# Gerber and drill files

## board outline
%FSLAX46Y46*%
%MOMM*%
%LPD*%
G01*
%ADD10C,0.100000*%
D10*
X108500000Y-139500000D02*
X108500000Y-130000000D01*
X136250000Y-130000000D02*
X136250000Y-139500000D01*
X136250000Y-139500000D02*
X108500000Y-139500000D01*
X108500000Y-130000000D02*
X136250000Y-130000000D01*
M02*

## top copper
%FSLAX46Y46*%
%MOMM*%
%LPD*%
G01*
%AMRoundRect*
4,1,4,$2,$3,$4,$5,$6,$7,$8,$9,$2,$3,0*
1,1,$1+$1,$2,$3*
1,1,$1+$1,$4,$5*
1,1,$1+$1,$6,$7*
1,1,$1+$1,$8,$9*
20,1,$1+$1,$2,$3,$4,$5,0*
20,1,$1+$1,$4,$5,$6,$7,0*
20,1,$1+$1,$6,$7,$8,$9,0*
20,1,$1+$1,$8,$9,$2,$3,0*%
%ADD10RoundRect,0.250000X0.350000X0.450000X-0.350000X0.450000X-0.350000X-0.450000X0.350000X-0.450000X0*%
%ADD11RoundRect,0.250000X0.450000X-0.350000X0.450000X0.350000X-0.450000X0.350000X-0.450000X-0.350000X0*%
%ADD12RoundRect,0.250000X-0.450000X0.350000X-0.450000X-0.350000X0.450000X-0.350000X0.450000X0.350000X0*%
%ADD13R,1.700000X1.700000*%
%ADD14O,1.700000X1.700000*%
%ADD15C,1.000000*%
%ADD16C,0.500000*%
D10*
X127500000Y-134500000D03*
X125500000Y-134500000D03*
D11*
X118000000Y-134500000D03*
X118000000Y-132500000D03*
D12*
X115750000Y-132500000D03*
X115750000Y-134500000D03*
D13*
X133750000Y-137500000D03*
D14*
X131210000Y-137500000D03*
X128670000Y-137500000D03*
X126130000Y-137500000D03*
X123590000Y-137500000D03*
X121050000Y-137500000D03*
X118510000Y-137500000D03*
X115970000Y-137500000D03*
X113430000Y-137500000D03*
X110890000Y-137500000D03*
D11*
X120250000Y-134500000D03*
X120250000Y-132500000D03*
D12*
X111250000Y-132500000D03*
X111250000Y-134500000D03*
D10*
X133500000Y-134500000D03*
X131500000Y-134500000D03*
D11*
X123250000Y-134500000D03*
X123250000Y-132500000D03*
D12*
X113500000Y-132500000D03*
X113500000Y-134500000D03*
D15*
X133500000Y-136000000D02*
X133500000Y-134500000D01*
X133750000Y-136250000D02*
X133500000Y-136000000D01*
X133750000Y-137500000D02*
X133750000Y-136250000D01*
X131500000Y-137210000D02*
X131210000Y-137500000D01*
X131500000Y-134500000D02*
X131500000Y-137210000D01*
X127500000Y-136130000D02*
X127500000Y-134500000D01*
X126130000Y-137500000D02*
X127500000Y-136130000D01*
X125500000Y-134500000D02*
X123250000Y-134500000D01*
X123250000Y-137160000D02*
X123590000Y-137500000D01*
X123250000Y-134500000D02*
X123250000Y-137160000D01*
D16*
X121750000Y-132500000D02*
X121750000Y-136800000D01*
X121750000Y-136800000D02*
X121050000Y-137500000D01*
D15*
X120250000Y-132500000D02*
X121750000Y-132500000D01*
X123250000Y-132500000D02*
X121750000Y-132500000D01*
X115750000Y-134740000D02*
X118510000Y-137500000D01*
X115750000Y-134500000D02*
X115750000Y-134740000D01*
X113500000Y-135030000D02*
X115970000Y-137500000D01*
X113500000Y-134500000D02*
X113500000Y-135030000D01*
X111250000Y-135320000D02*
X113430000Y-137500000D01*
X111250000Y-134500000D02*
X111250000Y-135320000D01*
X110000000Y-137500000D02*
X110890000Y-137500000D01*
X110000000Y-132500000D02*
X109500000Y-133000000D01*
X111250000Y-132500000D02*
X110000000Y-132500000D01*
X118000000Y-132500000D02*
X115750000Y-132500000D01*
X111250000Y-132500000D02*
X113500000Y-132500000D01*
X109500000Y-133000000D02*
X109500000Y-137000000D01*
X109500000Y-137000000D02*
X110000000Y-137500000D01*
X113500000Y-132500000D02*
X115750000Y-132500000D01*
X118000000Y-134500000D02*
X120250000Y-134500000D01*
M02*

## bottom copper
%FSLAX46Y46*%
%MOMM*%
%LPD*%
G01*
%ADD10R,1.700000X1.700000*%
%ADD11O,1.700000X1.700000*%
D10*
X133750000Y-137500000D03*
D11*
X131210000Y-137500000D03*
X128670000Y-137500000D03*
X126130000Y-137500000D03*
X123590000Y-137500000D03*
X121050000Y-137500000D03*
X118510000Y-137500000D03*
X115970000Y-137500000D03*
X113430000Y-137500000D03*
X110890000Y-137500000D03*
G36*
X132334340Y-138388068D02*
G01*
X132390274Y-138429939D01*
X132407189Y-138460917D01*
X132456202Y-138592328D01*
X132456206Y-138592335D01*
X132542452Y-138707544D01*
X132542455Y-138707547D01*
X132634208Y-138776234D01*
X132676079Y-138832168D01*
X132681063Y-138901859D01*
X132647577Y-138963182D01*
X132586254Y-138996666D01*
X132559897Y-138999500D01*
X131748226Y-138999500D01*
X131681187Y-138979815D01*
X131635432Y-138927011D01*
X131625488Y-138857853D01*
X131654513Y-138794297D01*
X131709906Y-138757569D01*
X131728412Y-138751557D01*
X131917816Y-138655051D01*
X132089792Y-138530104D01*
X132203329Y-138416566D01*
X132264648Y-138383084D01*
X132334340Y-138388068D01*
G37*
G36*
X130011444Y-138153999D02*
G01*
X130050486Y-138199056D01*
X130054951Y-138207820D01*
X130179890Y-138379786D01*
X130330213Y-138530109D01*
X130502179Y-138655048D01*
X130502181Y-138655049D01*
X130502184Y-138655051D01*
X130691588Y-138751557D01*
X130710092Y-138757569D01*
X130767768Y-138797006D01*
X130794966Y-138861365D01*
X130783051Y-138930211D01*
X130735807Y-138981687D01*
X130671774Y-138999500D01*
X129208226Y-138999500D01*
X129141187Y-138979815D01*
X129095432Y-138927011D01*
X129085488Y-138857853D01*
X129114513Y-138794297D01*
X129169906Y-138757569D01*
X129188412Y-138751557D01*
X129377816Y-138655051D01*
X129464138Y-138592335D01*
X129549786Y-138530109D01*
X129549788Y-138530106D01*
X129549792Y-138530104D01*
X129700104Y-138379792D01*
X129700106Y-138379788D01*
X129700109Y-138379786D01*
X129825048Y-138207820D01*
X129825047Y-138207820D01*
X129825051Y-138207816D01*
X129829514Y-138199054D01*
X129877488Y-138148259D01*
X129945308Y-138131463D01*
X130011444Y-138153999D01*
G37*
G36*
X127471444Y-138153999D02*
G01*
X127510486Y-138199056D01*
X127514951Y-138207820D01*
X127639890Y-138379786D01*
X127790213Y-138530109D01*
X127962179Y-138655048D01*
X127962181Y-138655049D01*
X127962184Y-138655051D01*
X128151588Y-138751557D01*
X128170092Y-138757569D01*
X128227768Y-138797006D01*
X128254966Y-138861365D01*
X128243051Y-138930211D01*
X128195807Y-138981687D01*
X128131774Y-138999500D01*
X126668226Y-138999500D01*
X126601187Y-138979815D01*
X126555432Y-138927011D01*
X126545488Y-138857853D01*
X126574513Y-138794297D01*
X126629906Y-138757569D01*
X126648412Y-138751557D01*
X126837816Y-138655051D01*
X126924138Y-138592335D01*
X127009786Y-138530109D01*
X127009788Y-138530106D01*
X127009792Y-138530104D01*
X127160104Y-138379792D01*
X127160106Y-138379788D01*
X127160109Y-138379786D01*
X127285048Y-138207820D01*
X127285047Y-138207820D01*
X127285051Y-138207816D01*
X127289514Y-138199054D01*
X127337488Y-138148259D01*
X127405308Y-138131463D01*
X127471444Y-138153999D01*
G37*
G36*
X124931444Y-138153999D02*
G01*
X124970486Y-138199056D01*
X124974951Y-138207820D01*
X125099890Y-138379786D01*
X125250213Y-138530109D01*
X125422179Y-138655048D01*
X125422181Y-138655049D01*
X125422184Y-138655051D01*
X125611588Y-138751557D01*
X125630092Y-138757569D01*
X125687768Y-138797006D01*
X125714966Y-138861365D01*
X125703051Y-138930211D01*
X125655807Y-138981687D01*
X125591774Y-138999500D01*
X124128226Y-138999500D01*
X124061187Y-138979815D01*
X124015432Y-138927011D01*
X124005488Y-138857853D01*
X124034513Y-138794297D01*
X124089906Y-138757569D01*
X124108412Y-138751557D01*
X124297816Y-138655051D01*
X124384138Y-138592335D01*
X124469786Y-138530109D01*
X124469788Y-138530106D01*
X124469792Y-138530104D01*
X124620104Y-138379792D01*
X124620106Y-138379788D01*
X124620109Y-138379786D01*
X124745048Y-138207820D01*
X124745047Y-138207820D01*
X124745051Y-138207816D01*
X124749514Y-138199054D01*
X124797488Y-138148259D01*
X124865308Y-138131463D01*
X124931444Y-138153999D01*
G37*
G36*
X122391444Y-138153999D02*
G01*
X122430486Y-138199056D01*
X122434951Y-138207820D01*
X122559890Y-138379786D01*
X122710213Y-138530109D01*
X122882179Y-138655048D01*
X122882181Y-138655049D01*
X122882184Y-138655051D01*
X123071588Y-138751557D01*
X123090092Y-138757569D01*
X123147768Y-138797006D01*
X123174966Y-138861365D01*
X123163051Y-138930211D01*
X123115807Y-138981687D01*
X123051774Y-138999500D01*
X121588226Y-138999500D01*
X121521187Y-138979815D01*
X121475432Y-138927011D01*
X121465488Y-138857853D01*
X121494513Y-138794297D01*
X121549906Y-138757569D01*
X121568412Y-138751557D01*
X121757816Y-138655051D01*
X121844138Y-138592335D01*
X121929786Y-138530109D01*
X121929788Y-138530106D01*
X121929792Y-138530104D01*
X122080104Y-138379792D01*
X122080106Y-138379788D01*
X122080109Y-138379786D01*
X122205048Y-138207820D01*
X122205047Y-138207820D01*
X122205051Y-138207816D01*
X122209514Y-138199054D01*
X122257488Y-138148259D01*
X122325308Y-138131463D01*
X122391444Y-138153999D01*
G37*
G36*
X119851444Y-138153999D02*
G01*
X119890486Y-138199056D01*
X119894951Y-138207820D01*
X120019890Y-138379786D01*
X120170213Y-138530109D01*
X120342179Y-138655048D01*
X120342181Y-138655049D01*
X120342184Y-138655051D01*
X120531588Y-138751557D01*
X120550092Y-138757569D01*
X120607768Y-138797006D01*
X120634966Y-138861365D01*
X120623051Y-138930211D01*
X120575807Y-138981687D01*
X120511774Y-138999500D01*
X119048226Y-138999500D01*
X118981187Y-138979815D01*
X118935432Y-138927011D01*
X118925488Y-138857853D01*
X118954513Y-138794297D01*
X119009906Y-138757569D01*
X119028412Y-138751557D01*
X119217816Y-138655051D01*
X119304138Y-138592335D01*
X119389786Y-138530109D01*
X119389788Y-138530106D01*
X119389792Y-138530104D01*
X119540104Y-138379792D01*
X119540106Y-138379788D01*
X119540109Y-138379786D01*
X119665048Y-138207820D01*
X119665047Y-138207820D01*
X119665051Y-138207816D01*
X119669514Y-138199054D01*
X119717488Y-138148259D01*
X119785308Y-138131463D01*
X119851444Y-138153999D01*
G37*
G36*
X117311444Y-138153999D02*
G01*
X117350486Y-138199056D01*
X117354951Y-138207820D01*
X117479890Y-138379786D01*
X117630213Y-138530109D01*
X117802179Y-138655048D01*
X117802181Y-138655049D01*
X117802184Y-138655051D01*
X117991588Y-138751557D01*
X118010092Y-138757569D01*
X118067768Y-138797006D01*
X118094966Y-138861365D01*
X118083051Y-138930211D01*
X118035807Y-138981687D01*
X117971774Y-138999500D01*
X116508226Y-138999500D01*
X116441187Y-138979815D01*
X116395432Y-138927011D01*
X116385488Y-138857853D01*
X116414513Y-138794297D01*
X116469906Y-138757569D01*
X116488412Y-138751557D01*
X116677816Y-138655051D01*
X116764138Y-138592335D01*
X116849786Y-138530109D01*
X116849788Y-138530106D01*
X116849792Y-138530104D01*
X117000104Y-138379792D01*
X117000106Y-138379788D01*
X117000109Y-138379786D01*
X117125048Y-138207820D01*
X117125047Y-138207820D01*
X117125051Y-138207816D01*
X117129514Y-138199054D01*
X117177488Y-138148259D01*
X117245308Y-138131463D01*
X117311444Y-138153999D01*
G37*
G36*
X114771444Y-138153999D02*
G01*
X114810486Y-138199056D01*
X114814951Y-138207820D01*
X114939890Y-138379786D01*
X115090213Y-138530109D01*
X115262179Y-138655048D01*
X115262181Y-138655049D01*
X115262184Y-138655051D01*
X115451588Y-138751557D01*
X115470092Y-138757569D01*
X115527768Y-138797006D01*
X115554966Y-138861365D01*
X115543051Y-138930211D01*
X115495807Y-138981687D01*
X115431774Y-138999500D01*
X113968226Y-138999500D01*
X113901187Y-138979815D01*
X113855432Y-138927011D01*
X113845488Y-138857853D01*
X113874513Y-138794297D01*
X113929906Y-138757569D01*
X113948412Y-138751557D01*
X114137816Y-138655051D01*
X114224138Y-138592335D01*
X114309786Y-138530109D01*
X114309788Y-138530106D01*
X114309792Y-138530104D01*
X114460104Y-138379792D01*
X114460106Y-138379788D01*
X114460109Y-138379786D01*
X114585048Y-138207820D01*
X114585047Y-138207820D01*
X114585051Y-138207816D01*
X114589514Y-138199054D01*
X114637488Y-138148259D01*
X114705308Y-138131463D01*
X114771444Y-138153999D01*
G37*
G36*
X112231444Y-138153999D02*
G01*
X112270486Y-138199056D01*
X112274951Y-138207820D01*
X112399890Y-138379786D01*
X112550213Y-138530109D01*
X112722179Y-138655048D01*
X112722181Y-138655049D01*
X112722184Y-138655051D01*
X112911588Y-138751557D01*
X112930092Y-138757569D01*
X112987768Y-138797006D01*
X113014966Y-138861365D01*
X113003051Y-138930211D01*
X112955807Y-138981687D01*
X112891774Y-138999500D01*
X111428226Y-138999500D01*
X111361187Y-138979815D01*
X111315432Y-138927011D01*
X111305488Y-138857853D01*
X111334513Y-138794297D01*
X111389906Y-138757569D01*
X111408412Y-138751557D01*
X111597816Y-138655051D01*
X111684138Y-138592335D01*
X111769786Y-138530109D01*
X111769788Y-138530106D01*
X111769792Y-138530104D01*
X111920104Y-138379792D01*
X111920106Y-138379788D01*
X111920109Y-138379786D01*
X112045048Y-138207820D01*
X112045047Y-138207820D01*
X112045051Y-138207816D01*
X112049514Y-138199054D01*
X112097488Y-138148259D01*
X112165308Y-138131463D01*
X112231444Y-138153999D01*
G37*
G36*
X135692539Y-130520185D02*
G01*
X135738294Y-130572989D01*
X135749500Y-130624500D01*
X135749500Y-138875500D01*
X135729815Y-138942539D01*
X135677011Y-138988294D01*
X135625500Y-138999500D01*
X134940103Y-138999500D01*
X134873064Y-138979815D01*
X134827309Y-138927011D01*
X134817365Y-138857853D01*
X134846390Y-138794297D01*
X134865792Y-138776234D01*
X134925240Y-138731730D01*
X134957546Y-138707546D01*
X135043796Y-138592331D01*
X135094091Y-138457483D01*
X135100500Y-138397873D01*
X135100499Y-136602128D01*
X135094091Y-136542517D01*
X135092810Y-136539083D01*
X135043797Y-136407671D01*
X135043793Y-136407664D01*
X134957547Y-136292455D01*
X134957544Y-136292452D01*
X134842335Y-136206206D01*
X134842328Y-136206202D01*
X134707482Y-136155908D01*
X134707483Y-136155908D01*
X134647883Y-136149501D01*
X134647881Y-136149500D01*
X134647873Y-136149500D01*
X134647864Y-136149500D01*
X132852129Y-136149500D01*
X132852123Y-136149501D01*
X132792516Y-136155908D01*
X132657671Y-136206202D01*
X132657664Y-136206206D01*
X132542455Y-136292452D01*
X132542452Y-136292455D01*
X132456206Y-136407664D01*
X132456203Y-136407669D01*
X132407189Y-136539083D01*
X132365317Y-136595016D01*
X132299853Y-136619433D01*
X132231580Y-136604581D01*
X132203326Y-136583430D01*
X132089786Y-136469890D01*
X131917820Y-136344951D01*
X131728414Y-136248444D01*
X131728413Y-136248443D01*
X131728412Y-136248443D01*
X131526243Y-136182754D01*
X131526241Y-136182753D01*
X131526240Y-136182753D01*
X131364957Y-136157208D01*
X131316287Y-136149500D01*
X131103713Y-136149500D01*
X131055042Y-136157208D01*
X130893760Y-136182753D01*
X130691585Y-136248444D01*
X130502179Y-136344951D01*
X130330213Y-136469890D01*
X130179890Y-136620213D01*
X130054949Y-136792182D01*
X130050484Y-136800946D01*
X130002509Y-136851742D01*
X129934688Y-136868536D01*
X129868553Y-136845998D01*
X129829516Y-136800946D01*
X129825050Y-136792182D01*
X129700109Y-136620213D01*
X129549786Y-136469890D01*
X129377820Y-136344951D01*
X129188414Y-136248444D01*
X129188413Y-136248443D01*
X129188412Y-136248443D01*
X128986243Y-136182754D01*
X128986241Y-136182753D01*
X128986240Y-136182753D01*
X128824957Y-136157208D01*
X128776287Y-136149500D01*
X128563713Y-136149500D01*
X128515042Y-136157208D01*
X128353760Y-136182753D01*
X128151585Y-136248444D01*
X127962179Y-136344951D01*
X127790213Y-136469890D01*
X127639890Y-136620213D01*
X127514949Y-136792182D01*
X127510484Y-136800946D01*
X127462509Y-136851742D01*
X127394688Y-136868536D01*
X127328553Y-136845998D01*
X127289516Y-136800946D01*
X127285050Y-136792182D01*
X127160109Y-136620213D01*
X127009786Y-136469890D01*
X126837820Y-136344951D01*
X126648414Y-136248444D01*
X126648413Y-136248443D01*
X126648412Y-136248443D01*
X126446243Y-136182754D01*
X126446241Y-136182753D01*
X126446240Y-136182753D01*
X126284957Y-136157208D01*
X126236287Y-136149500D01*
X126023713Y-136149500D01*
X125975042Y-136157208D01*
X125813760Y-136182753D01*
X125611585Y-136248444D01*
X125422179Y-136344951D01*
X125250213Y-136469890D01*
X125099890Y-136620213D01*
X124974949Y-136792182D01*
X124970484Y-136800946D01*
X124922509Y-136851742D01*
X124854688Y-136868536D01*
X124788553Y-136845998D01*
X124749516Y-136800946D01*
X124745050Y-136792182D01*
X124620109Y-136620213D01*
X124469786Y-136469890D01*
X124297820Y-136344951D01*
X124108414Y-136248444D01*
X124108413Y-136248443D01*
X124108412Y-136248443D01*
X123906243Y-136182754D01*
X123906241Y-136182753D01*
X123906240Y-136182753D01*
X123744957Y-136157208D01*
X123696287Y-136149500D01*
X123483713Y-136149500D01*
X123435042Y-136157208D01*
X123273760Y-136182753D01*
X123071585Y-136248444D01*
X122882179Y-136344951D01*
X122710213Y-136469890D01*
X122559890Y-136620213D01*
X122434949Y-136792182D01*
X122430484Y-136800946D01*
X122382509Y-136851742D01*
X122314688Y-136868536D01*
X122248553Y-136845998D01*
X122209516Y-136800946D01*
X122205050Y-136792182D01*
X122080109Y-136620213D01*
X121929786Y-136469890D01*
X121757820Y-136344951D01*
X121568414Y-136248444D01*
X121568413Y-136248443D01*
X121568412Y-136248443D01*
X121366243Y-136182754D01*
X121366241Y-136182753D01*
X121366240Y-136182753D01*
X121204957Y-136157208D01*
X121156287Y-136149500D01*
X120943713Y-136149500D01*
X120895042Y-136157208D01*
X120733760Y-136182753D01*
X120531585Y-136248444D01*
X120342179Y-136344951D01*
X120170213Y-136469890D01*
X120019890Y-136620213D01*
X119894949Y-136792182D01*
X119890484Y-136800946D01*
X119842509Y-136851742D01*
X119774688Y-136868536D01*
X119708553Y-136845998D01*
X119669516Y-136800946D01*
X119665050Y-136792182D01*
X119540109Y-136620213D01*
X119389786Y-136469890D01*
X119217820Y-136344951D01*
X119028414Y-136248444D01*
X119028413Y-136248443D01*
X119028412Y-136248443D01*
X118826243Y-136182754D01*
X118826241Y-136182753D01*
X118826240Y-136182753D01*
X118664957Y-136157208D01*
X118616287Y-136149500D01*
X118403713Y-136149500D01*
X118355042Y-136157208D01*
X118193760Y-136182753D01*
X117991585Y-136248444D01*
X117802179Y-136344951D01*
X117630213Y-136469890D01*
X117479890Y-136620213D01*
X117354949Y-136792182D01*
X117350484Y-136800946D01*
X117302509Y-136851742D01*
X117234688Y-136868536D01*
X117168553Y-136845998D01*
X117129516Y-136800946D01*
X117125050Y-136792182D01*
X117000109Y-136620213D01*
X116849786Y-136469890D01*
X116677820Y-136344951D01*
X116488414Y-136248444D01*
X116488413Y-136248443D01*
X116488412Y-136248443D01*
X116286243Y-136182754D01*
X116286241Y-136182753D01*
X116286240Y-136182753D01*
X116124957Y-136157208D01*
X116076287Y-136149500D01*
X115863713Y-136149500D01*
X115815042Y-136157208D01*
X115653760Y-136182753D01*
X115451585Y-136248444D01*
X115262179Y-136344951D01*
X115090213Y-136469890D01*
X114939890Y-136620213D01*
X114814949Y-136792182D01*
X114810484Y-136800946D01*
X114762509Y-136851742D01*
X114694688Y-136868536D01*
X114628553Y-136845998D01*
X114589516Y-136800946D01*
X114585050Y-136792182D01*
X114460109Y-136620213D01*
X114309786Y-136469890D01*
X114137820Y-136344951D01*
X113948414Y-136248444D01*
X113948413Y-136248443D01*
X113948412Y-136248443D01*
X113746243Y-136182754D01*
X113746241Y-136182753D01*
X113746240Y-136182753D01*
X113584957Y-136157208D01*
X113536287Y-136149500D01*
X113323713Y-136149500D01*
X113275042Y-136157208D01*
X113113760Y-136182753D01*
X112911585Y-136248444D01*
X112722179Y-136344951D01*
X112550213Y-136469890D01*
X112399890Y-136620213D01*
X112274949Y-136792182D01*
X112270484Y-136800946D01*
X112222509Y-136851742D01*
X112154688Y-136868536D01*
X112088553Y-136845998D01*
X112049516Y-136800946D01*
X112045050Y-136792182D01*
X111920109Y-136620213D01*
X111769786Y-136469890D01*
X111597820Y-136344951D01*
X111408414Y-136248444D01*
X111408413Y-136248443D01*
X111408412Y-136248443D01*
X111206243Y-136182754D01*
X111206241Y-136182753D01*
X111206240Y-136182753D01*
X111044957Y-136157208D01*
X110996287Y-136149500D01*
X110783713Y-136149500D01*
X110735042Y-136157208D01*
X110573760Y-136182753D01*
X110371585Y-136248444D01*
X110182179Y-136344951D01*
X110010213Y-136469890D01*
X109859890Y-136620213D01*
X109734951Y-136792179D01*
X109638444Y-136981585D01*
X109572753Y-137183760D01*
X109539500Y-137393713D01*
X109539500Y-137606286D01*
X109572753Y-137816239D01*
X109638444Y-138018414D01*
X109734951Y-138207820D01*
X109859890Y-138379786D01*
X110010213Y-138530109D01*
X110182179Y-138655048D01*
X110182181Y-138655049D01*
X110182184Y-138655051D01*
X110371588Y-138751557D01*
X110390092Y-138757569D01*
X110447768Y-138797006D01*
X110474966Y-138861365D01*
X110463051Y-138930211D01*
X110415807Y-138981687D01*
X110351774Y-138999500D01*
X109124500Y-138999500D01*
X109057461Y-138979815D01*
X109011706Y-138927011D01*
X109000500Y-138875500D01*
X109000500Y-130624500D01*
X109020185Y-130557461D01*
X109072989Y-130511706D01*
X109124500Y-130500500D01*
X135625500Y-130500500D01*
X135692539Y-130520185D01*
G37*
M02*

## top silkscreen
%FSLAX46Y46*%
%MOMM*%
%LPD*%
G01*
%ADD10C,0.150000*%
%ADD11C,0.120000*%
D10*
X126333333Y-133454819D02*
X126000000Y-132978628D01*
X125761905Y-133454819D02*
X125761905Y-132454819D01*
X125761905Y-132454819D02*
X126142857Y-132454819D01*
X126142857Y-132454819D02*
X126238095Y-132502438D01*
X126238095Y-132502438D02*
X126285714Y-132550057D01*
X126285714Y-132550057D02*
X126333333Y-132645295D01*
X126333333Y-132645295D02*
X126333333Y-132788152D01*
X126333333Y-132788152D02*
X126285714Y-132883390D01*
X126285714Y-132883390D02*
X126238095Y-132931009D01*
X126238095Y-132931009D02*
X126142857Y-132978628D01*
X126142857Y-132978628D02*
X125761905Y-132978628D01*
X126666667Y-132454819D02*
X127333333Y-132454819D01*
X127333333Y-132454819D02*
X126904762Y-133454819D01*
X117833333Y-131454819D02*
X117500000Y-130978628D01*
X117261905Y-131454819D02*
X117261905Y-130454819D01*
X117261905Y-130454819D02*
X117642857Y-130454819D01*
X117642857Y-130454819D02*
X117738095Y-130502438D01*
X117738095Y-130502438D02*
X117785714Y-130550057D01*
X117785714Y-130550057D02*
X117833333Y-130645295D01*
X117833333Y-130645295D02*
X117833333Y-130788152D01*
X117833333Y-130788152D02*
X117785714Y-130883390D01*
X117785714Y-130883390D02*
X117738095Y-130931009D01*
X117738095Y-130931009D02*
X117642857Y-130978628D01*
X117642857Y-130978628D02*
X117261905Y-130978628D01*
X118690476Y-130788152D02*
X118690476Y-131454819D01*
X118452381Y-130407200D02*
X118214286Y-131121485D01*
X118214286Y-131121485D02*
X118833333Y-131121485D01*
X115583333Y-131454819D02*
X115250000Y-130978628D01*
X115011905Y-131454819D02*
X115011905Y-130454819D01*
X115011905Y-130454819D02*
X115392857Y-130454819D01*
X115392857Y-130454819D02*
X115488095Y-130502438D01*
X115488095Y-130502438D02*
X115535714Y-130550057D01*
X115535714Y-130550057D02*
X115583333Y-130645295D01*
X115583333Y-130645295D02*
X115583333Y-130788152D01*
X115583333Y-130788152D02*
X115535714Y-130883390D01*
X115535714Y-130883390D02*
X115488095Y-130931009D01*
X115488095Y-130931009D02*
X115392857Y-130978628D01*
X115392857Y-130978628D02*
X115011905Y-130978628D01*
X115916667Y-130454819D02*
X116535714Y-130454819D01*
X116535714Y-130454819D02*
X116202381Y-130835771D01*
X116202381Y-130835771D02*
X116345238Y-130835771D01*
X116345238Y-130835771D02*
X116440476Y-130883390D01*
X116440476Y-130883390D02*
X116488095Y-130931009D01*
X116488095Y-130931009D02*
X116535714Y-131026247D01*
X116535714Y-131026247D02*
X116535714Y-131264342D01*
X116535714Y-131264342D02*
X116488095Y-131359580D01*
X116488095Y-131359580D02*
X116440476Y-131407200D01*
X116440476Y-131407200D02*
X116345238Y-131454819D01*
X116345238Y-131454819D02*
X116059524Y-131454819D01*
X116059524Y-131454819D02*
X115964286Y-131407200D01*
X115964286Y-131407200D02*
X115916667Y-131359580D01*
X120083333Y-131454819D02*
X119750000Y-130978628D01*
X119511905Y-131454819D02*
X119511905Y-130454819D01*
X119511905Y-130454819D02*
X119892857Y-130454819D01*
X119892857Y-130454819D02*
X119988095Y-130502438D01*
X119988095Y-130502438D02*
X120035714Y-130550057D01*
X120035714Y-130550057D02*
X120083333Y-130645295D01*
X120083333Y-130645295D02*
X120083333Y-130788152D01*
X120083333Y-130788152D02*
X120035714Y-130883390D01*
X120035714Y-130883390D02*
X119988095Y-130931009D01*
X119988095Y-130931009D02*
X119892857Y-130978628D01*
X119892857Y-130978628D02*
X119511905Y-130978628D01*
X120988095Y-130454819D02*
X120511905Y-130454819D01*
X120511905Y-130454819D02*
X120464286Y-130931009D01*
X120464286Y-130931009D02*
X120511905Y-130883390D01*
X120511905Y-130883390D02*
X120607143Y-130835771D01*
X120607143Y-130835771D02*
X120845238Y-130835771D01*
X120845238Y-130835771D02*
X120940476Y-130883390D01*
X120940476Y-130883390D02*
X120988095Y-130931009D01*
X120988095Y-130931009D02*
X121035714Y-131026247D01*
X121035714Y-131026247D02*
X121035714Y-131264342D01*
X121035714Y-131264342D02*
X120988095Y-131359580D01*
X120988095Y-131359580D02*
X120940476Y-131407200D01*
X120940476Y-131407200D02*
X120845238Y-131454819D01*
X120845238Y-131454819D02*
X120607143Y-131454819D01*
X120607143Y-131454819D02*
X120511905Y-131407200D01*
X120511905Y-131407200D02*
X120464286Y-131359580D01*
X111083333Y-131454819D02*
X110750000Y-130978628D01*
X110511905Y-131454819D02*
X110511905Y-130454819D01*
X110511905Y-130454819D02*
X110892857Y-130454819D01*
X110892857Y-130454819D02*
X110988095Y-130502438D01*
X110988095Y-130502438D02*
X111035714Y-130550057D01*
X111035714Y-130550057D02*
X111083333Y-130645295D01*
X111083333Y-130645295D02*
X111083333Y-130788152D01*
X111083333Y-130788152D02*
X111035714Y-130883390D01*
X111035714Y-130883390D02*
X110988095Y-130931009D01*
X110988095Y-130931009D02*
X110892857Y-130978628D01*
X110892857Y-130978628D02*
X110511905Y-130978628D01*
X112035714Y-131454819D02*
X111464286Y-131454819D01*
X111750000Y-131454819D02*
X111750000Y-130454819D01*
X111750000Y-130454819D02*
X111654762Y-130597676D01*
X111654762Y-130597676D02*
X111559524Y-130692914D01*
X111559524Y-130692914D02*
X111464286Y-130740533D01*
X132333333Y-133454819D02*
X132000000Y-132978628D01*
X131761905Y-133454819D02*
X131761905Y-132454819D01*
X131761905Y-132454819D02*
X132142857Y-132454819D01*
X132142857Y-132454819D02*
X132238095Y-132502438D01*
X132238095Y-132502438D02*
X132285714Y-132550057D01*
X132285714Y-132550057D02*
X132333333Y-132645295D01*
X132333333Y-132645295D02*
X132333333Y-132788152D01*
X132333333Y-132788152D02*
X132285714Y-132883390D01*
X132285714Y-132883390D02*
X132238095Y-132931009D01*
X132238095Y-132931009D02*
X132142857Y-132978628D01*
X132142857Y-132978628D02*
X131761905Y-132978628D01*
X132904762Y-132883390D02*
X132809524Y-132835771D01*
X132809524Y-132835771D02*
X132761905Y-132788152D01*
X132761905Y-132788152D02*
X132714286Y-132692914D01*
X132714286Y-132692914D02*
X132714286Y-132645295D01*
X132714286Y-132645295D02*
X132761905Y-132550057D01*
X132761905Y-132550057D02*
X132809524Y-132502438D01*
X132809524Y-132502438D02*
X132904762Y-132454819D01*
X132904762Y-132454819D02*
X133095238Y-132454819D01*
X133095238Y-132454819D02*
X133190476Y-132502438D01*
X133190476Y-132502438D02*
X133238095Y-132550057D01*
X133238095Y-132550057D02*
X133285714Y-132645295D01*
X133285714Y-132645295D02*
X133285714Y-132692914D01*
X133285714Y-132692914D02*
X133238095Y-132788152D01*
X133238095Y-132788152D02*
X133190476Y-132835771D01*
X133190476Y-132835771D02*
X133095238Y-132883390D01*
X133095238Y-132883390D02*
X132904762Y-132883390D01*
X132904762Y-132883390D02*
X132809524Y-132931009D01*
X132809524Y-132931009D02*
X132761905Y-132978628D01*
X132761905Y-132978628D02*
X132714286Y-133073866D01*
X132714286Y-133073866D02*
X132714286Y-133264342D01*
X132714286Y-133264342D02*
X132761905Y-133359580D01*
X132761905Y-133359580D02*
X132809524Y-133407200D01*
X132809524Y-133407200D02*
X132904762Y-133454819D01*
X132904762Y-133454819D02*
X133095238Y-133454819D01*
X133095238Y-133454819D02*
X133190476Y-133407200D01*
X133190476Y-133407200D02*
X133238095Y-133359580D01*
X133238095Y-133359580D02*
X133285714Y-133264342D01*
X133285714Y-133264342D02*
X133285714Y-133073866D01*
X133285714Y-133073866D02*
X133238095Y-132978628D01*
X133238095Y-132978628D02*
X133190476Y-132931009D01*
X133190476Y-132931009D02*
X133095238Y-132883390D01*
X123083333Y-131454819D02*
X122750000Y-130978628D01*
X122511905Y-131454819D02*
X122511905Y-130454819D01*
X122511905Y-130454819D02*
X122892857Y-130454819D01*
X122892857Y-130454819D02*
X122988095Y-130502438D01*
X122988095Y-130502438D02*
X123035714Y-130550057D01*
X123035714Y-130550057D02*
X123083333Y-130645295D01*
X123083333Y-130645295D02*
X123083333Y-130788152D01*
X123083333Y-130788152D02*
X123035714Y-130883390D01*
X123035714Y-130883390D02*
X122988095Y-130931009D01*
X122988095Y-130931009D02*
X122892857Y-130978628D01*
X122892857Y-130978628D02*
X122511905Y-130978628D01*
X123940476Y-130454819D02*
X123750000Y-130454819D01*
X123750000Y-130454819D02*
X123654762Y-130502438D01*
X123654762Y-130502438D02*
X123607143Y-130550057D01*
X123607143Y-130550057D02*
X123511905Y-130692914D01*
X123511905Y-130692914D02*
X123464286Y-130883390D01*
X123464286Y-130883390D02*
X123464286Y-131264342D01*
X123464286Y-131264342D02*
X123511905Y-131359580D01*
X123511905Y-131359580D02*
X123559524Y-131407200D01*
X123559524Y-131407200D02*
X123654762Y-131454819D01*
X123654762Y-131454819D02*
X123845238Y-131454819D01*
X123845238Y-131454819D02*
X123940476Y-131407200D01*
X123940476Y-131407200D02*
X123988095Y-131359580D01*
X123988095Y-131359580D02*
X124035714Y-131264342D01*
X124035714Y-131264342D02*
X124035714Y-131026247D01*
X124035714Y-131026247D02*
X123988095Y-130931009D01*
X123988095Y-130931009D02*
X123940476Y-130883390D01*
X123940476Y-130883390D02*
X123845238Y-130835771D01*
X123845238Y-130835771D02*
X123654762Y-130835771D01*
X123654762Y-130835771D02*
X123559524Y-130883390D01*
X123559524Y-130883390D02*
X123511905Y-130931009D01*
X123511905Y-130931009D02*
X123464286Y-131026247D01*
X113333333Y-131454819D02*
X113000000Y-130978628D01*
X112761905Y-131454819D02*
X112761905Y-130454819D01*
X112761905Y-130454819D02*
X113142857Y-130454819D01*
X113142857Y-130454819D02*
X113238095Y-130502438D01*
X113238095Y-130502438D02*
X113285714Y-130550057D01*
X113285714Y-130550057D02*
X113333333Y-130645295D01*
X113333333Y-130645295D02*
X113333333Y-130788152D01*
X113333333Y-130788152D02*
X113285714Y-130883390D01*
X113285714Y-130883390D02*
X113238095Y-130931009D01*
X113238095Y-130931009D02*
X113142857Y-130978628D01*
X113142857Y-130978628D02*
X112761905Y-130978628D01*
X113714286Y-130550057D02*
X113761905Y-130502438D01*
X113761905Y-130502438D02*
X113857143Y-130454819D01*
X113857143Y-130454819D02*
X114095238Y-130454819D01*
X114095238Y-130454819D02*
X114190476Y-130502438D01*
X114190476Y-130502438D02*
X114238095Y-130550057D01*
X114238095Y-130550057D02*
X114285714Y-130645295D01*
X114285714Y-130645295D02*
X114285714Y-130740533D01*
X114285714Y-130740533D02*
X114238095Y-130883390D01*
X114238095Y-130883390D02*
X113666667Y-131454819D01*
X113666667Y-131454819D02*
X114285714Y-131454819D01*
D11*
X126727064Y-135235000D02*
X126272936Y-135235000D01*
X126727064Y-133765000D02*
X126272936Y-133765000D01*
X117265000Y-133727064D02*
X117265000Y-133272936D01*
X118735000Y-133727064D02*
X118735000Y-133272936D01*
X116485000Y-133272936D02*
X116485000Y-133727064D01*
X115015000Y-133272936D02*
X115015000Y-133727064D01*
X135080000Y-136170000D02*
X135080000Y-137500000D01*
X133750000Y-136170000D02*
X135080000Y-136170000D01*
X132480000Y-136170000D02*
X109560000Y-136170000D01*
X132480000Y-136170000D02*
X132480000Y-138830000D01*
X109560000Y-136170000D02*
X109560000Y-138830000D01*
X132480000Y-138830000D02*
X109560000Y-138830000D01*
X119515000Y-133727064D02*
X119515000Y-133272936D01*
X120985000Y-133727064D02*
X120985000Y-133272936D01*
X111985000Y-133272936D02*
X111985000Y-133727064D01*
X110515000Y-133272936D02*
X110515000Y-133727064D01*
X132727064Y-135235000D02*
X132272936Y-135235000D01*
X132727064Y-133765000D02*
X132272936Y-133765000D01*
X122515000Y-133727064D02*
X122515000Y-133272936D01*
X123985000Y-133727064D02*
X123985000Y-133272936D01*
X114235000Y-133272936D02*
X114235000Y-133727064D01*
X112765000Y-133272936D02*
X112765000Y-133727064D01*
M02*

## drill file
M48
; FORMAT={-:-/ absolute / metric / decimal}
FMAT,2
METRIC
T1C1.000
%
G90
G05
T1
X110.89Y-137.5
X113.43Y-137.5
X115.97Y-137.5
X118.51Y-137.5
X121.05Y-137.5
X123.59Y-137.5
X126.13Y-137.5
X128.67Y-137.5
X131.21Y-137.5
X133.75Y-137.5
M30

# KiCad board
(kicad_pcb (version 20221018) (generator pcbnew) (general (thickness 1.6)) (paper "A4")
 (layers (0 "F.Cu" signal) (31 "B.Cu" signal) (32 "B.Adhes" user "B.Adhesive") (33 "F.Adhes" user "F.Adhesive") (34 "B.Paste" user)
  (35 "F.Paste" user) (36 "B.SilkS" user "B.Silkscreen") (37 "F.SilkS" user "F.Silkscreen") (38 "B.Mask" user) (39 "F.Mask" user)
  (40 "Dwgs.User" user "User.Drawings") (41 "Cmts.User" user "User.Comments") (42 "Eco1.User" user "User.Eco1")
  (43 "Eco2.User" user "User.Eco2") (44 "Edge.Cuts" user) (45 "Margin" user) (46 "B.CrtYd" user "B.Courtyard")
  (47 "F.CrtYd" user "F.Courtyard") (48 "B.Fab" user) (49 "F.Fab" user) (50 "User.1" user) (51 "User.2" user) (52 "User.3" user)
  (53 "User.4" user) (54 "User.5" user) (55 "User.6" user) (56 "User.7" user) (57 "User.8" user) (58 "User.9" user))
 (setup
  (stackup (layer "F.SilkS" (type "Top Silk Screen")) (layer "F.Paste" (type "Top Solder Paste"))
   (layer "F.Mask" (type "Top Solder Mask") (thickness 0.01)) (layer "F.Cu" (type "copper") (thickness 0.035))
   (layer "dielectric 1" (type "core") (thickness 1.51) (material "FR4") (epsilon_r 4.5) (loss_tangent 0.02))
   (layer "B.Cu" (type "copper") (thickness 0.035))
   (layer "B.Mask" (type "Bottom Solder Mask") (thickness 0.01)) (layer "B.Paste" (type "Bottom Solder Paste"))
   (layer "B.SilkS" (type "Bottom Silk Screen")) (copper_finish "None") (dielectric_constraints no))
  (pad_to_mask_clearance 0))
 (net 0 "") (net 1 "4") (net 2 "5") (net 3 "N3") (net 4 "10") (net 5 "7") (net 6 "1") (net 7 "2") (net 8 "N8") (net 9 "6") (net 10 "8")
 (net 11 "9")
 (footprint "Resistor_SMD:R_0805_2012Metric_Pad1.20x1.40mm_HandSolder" (layer "F.Cu") (at 126.5 134.5 180)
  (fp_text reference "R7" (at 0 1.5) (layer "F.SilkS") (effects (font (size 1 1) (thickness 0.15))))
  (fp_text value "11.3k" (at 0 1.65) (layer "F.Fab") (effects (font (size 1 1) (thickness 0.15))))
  (fp_line (start -0.227064 -0.735) (end 0.227064 -0.735) (stroke (width 0.12) (type solid)) (layer "F.SilkS"))
  (fp_line (start -0.227064 0.735) (end 0.227064 0.735) (stroke (width 0.12) (type solid)) (layer "F.SilkS"))
  (pad "1" smd roundrect (at -1 0 180) (size 1.2 1.4) (layers "F.Cu" "F.Paste" "F.Mask") (roundrect_rratio 0.2083333333) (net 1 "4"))
  (pad "2" smd roundrect (at 1 0 180) (size 1.2 1.4) (layers "F.Cu" "F.Paste" "F.Mask") (roundrect_rratio 0.2083333333) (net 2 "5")))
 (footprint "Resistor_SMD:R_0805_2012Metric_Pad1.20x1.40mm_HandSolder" (layer "F.Cu") (at 118 133.5 90)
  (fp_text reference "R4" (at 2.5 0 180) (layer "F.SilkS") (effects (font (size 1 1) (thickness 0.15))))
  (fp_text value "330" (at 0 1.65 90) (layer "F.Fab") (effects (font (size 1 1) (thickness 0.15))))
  (fp_line (start -0.227064 -0.735) (end 0.227064 -0.735) (stroke (width 0.12) (type solid)) (layer "F.SilkS"))
  (fp_line (start -0.227064 0.735) (end 0.227064 0.735) (stroke (width 0.12) (type solid)) (layer "F.SilkS"))
  (pad "1" smd roundrect (at -1 0 90) (size 1.2 1.4) (layers "F.Cu" "F.Paste" "F.Mask") (roundrect_rratio 0.2083333333) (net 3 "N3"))
  (pad "2" smd roundrect (at 1 0 90) (size 1.2 1.4) (layers "F.Cu" "F.Paste" "F.Mask") (roundrect_rratio 0.2083333333) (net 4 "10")))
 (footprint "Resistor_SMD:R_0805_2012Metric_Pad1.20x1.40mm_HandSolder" (layer "F.Cu") (at 115.75 133.5 -90)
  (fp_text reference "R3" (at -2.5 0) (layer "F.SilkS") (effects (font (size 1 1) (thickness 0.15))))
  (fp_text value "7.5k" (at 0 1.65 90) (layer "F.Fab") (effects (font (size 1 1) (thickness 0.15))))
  (fp_line (start -0.227064 -0.735) (end 0.227064 -0.735) (stroke (width 0.12) (type solid)) (layer "F.SilkS"))
  (fp_line (start -0.227064 0.735) (end 0.227064 0.735) (stroke (width 0.12) (type solid)) (layer "F.SilkS"))
  (pad "1" smd roundrect (at -1 0 270) (size 1.2 1.4) (layers "F.Cu" "F.Paste" "F.Mask") (roundrect_rratio 0.2083333333) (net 4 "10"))
  (pad "2" smd roundrect (at 1 0 270) (size 1.2 1.4) (layers "F.Cu" "F.Paste" "F.Mask") (roundrect_rratio 0.2083333333) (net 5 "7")))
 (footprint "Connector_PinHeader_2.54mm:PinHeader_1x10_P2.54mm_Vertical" (layer "F.Cu") (at 133.75 137.5 -90)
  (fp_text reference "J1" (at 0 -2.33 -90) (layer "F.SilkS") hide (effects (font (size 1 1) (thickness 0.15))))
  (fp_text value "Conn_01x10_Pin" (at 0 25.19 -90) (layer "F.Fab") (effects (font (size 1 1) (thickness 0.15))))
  (fp_line (start -1.33 -1.33) (end 0 -1.33) (stroke (width 0.12) (type solid)) (layer "F.SilkS"))
  (fp_line (start -1.33 0) (end -1.33 -1.33) (stroke (width 0.12) (type solid)) (layer "F.SilkS"))
  (fp_line (start -1.33 1.27) (end -1.33 24.19) (stroke (width 0.12) (type solid)) (layer "F.SilkS"))
  (fp_line (start -1.33 1.27) (end 1.33 1.27) (stroke (width 0.12) (type solid)) (layer "F.SilkS"))
  (fp_line (start -1.33 24.19) (end 1.33 24.19) (stroke (width 0.12) (type solid)) (layer "F.SilkS"))
  (fp_line (start 1.33 1.27) (end 1.33 24.19) (stroke (width 0.12) (type solid)) (layer "F.SilkS"))
  (pad "1" thru_hole rect (at 0 0 270) (size 1.7 1.7) (drill 1) (layers "*.Cu" "*.Mask") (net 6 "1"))
  (pad "2" thru_hole oval (at 0 2.54 270) (size 1.7 1.7) (drill 1) (layers "*.Cu" "*.Mask") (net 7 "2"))
  (pad "3" thru_hole oval (at 0 5.08 270) (size 1.7 1.7) (drill 1) (layers "*.Cu" "*.Mask") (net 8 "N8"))
  (pad "4" thru_hole oval (at 0 7.62 270) (size 1.7 1.7) (drill 1) (layers "*.Cu" "*.Mask") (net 1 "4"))
  (pad "5" thru_hole oval (at 0 10.16 270) (size 1.7 1.7) (drill 1) (layers "*.Cu" "*.Mask") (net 2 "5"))
  (pad "6" thru_hole oval (at 0 12.7 270) (size 1.7 1.7) (drill 1) (layers "*.Cu" "*.Mask") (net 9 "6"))
  (pad "7" thru_hole oval (at 0 15.24 270) (size 1.7 1.7) (drill 1) (layers "*.Cu" "*.Mask") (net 5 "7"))
  (pad "8" thru_hole oval (at 0 17.78 270) (size 1.7 1.7) (drill 1) (layers "*.Cu" "*.Mask") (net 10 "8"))
  (pad "9" thru_hole oval (at 0 20.32 270) (size 1.7 1.7) (drill 1) (layers "*.Cu" "*.Mask") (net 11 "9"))
  (pad "10" thru_hole oval (at 0 22.86 270) (size 1.7 1.7) (drill 1) (layers "*.Cu" "*.Mask") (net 4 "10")))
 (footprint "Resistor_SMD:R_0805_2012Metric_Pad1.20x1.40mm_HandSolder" (layer "F.Cu") (at 120.25 133.5 90)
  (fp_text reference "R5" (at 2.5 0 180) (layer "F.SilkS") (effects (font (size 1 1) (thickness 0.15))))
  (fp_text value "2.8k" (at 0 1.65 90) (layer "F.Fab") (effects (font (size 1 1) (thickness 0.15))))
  (fp_line (start -0.227064 -0.735) (end 0.227064 -0.735) (stroke (width 0.12) (type solid)) (layer "F.SilkS"))
  (fp_line (start -0.227064 0.735) (end 0.227064 0.735) (stroke (width 0.12) (type solid)) (layer "F.SilkS"))
  (pad "1" smd roundrect (at -1 0 90) (size 1.2 1.4) (layers "F.Cu" "F.Paste" "F.Mask") (roundrect_rratio 0.2083333333) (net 3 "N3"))
  (pad "2" smd roundrect (at 1 0 90) (size 1.2 1.4) (layers "F.Cu" "F.Paste" "F.Mask") (roundrect_rratio 0.2083333333) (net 9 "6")))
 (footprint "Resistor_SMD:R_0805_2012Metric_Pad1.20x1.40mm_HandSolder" (layer "F.Cu") (at 111.25 133.5 -90)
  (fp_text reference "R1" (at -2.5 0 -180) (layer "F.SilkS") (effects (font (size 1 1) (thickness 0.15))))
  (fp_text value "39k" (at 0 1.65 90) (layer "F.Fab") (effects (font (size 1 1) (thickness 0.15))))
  (fp_line (start -0.227064 -0.735) (end 0.227064 -0.735) (stroke (width 0.12) (type solid)) (layer "F.SilkS"))
  (fp_line (start -0.227064 0.735) (end 0.227064 0.735) (stroke (width 0.12) (type solid)) (layer "F.SilkS"))
  (pad "1" smd roundrect (at -1 0 270) (size 1.2 1.4) (layers "F.Cu" "F.Paste" "F.Mask") (roundrect_rratio 0.2083333333) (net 4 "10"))
  (pad "2" smd roundrect (at 1 0 270) (size 1.2 1.4) (layers "F.Cu" "F.Paste" "F.Mask") (roundrect_rratio 0.2083333333) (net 11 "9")))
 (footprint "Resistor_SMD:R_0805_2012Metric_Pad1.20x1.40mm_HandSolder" (layer "F.Cu") (at 132.5 134.5 180)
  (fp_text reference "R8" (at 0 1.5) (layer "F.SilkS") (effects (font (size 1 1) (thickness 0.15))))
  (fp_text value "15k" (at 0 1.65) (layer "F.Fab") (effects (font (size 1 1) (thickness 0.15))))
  (fp_line (start -0.227064 -0.735) (end 0.227064 -0.735) (stroke (width 0.12) (type solid)) (layer "F.SilkS"))
  (fp_line (start -0.227064 0.735) (end 0.227064 0.735) (stroke (width 0.12) (type solid)) (layer "F.SilkS"))
  (pad "1" smd roundrect (at -1 0 180) (size 1.2 1.4) (layers "F.Cu" "F.Paste" "F.Mask") (roundrect_rratio 0.2083333333) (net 6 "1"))
  (pad "2" smd roundrect (at 1 0 180) (size 1.2 1.4) (layers "F.Cu" "F.Paste" "F.Mask") (roundrect_rratio 0.2083333333) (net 7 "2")))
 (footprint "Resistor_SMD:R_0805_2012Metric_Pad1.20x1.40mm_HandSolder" (layer "F.Cu") (at 123.25 133.5 90)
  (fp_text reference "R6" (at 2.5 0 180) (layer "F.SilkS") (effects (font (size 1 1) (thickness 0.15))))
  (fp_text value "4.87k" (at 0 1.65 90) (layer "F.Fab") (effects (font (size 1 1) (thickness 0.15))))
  (fp_line (start -0.227064 -0.735) (end 0.227064 -0.735) (stroke (width 0.12) (type solid)) (layer "F.SilkS"))
  (fp_line (start -0.227064 0.735) (end 0.227064 0.735) (stroke (width 0.12) (type solid)) (layer "F.SilkS"))
  (pad "1" smd roundrect (at -1 0 90) (size 1.2 1.4) (layers "F.Cu" "F.Paste" "F.Mask") (roundrect_rratio 0.2083333333) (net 2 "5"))
  (pad "2" smd roundrect (at 1 0 90) (size 1.2 1.4) (layers "F.Cu" "F.Paste" "F.Mask") (roundrect_rratio 0.2083333333) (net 9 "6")))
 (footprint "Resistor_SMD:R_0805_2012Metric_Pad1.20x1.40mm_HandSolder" (layer "F.Cu") (at 113.5 133.5 -90)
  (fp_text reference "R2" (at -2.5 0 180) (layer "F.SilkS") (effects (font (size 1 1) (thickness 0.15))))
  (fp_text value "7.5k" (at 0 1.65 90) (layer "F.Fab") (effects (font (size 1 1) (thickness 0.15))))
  (fp_line (start -0.227064 -0.735) (end 0.227064 -0.735) (stroke (width 0.12) (type solid)) (layer "F.SilkS"))
  (fp_line (start -0.227064 0.735) (end 0.227064 0.735) (stroke (width 0.12) (type solid)) (layer "F.SilkS"))
  (pad "1" smd roundrect (at -1 0 270) (size 1.2 1.4) (layers "F.Cu" "F.Paste" "F.Mask") (roundrect_rratio 0.2083333333) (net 4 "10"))
  (pad "2" smd roundrect (at 1 0 270) (size 1.2 1.4) (layers "F.Cu" "F.Paste" "F.Mask") (roundrect_rratio 0.2083333333) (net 10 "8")))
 (gr_line (start 108.5 139.5) (end 108.5 130) (stroke (width 0.1) (type default)) (layer "Edge.Cuts"))
 (gr_line (start 136.25 130) (end 136.25 139.5) (stroke (width 0.1) (type default)) (layer "Edge.Cuts"))
 (gr_line (start 136.25 139.5) (end 108.5 139.5) (stroke (width 0.1) (type default)) (layer "Edge.Cuts"))
 (gr_line (start 108.5 130) (end 136.25 130) (stroke (width 0.1) (type default)) (layer "Edge.Cuts"))
 (segment (start 133.5 136) (end 133.5 134.5) (width 1) (layer "F.Cu") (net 6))
 (segment (start 133.75 136.25) (end 133.5 136) (width 1) (layer "F.Cu") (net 6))
 (segment (start 133.75 137.5) (end 133.75 136.25) (width 1) (layer "F.Cu") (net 6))
 (segment (start 131.5 137.21) (end 131.21 137.5) (width 1) (layer "F.Cu") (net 7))
 (segment (start 131.5 134.5) (end 131.5 137.21) (width 1) (layer "F.Cu") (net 7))
 (segment (start 127.5 136.13) (end 127.5 134.5) (width 1) (layer "F.Cu") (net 1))
 (segment (start 126.13 137.5) (end 127.5 136.13) (width 1) (layer "F.Cu") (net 1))
 (segment (start 125.5 134.5) (end 123.25 134.5) (width 1) (layer "F.Cu") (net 2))
 (segment (start 123.25 137.16) (end 123.59 137.5) (width 1) (layer "F.Cu") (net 2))
 (segment (start 123.25 134.5) (end 123.25 137.16) (width 1) (layer "F.Cu") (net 2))
 (segment (start 121.75 132.5) (end 121.75 136.8) (width 0.5) (layer "F.Cu") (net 9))
 (segment (start 121.75 136.8) (end 121.05 137.5) (width 0.5) (layer "F.Cu") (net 9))
 (segment (start 120.25 132.5) (end 121.75 132.5) (width 1) (layer "F.Cu") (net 9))
 (segment (start 123.25 132.5) (end 121.75 132.5) (width 1) (layer "F.Cu") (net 9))
 (segment (start 115.75 134.74) (end 118.51 137.5) (width 1) (layer "F.Cu") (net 5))
 (segment (start 115.75 134.5) (end 115.75 134.74) (width 1) (layer "F.Cu") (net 5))
 (segment (start 113.5 135.03) (end 115.97 137.5) (width 1) (layer "F.Cu") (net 10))
 (segment (start 113.5 134.5) (end 113.5 135.03) (width 1) (layer "F.Cu") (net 10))
 (segment (start 111.25 135.32) (end 113.43 137.5) (width 1) (layer "F.Cu") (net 11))
 (segment (start 111.25 134.5) (end 111.25 135.32) (width 1) (layer "F.Cu") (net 11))
 (segment (start 110 137.5) (end 110.89 137.5) (width 1) (layer "F.Cu") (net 4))
 (segment (start 110 132.5) (end 109.5 133) (width 1) (layer "F.Cu") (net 4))
 (segment (start 111.25 132.5) (end 110 132.5) (width 1) (layer "F.Cu") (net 4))
 (segment (start 118 132.5) (end 115.75 132.5) (width 1) (layer "F.Cu") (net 4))
 (segment (start 111.25 132.5) (end 113.5 132.5) (width 1) (layer "F.Cu") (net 4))
 (segment (start 109.5 133) (end 109.5 137) (width 1) (layer "F.Cu") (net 4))
 (segment (start 109.5 137) (end 110 137.5) (width 1) (layer "F.Cu") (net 4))
 (segment (start 113.5 132.5) (end 115.75 132.5) (width 1) (layer "F.Cu") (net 4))
 (segment (start 118 134.5) (end 120.25 134.5) (width 1) (layer "F.Cu") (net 3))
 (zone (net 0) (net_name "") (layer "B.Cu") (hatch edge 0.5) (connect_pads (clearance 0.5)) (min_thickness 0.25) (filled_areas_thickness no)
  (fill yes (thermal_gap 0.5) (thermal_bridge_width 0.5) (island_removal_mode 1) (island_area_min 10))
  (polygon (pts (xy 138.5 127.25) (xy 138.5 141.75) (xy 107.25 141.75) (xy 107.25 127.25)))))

